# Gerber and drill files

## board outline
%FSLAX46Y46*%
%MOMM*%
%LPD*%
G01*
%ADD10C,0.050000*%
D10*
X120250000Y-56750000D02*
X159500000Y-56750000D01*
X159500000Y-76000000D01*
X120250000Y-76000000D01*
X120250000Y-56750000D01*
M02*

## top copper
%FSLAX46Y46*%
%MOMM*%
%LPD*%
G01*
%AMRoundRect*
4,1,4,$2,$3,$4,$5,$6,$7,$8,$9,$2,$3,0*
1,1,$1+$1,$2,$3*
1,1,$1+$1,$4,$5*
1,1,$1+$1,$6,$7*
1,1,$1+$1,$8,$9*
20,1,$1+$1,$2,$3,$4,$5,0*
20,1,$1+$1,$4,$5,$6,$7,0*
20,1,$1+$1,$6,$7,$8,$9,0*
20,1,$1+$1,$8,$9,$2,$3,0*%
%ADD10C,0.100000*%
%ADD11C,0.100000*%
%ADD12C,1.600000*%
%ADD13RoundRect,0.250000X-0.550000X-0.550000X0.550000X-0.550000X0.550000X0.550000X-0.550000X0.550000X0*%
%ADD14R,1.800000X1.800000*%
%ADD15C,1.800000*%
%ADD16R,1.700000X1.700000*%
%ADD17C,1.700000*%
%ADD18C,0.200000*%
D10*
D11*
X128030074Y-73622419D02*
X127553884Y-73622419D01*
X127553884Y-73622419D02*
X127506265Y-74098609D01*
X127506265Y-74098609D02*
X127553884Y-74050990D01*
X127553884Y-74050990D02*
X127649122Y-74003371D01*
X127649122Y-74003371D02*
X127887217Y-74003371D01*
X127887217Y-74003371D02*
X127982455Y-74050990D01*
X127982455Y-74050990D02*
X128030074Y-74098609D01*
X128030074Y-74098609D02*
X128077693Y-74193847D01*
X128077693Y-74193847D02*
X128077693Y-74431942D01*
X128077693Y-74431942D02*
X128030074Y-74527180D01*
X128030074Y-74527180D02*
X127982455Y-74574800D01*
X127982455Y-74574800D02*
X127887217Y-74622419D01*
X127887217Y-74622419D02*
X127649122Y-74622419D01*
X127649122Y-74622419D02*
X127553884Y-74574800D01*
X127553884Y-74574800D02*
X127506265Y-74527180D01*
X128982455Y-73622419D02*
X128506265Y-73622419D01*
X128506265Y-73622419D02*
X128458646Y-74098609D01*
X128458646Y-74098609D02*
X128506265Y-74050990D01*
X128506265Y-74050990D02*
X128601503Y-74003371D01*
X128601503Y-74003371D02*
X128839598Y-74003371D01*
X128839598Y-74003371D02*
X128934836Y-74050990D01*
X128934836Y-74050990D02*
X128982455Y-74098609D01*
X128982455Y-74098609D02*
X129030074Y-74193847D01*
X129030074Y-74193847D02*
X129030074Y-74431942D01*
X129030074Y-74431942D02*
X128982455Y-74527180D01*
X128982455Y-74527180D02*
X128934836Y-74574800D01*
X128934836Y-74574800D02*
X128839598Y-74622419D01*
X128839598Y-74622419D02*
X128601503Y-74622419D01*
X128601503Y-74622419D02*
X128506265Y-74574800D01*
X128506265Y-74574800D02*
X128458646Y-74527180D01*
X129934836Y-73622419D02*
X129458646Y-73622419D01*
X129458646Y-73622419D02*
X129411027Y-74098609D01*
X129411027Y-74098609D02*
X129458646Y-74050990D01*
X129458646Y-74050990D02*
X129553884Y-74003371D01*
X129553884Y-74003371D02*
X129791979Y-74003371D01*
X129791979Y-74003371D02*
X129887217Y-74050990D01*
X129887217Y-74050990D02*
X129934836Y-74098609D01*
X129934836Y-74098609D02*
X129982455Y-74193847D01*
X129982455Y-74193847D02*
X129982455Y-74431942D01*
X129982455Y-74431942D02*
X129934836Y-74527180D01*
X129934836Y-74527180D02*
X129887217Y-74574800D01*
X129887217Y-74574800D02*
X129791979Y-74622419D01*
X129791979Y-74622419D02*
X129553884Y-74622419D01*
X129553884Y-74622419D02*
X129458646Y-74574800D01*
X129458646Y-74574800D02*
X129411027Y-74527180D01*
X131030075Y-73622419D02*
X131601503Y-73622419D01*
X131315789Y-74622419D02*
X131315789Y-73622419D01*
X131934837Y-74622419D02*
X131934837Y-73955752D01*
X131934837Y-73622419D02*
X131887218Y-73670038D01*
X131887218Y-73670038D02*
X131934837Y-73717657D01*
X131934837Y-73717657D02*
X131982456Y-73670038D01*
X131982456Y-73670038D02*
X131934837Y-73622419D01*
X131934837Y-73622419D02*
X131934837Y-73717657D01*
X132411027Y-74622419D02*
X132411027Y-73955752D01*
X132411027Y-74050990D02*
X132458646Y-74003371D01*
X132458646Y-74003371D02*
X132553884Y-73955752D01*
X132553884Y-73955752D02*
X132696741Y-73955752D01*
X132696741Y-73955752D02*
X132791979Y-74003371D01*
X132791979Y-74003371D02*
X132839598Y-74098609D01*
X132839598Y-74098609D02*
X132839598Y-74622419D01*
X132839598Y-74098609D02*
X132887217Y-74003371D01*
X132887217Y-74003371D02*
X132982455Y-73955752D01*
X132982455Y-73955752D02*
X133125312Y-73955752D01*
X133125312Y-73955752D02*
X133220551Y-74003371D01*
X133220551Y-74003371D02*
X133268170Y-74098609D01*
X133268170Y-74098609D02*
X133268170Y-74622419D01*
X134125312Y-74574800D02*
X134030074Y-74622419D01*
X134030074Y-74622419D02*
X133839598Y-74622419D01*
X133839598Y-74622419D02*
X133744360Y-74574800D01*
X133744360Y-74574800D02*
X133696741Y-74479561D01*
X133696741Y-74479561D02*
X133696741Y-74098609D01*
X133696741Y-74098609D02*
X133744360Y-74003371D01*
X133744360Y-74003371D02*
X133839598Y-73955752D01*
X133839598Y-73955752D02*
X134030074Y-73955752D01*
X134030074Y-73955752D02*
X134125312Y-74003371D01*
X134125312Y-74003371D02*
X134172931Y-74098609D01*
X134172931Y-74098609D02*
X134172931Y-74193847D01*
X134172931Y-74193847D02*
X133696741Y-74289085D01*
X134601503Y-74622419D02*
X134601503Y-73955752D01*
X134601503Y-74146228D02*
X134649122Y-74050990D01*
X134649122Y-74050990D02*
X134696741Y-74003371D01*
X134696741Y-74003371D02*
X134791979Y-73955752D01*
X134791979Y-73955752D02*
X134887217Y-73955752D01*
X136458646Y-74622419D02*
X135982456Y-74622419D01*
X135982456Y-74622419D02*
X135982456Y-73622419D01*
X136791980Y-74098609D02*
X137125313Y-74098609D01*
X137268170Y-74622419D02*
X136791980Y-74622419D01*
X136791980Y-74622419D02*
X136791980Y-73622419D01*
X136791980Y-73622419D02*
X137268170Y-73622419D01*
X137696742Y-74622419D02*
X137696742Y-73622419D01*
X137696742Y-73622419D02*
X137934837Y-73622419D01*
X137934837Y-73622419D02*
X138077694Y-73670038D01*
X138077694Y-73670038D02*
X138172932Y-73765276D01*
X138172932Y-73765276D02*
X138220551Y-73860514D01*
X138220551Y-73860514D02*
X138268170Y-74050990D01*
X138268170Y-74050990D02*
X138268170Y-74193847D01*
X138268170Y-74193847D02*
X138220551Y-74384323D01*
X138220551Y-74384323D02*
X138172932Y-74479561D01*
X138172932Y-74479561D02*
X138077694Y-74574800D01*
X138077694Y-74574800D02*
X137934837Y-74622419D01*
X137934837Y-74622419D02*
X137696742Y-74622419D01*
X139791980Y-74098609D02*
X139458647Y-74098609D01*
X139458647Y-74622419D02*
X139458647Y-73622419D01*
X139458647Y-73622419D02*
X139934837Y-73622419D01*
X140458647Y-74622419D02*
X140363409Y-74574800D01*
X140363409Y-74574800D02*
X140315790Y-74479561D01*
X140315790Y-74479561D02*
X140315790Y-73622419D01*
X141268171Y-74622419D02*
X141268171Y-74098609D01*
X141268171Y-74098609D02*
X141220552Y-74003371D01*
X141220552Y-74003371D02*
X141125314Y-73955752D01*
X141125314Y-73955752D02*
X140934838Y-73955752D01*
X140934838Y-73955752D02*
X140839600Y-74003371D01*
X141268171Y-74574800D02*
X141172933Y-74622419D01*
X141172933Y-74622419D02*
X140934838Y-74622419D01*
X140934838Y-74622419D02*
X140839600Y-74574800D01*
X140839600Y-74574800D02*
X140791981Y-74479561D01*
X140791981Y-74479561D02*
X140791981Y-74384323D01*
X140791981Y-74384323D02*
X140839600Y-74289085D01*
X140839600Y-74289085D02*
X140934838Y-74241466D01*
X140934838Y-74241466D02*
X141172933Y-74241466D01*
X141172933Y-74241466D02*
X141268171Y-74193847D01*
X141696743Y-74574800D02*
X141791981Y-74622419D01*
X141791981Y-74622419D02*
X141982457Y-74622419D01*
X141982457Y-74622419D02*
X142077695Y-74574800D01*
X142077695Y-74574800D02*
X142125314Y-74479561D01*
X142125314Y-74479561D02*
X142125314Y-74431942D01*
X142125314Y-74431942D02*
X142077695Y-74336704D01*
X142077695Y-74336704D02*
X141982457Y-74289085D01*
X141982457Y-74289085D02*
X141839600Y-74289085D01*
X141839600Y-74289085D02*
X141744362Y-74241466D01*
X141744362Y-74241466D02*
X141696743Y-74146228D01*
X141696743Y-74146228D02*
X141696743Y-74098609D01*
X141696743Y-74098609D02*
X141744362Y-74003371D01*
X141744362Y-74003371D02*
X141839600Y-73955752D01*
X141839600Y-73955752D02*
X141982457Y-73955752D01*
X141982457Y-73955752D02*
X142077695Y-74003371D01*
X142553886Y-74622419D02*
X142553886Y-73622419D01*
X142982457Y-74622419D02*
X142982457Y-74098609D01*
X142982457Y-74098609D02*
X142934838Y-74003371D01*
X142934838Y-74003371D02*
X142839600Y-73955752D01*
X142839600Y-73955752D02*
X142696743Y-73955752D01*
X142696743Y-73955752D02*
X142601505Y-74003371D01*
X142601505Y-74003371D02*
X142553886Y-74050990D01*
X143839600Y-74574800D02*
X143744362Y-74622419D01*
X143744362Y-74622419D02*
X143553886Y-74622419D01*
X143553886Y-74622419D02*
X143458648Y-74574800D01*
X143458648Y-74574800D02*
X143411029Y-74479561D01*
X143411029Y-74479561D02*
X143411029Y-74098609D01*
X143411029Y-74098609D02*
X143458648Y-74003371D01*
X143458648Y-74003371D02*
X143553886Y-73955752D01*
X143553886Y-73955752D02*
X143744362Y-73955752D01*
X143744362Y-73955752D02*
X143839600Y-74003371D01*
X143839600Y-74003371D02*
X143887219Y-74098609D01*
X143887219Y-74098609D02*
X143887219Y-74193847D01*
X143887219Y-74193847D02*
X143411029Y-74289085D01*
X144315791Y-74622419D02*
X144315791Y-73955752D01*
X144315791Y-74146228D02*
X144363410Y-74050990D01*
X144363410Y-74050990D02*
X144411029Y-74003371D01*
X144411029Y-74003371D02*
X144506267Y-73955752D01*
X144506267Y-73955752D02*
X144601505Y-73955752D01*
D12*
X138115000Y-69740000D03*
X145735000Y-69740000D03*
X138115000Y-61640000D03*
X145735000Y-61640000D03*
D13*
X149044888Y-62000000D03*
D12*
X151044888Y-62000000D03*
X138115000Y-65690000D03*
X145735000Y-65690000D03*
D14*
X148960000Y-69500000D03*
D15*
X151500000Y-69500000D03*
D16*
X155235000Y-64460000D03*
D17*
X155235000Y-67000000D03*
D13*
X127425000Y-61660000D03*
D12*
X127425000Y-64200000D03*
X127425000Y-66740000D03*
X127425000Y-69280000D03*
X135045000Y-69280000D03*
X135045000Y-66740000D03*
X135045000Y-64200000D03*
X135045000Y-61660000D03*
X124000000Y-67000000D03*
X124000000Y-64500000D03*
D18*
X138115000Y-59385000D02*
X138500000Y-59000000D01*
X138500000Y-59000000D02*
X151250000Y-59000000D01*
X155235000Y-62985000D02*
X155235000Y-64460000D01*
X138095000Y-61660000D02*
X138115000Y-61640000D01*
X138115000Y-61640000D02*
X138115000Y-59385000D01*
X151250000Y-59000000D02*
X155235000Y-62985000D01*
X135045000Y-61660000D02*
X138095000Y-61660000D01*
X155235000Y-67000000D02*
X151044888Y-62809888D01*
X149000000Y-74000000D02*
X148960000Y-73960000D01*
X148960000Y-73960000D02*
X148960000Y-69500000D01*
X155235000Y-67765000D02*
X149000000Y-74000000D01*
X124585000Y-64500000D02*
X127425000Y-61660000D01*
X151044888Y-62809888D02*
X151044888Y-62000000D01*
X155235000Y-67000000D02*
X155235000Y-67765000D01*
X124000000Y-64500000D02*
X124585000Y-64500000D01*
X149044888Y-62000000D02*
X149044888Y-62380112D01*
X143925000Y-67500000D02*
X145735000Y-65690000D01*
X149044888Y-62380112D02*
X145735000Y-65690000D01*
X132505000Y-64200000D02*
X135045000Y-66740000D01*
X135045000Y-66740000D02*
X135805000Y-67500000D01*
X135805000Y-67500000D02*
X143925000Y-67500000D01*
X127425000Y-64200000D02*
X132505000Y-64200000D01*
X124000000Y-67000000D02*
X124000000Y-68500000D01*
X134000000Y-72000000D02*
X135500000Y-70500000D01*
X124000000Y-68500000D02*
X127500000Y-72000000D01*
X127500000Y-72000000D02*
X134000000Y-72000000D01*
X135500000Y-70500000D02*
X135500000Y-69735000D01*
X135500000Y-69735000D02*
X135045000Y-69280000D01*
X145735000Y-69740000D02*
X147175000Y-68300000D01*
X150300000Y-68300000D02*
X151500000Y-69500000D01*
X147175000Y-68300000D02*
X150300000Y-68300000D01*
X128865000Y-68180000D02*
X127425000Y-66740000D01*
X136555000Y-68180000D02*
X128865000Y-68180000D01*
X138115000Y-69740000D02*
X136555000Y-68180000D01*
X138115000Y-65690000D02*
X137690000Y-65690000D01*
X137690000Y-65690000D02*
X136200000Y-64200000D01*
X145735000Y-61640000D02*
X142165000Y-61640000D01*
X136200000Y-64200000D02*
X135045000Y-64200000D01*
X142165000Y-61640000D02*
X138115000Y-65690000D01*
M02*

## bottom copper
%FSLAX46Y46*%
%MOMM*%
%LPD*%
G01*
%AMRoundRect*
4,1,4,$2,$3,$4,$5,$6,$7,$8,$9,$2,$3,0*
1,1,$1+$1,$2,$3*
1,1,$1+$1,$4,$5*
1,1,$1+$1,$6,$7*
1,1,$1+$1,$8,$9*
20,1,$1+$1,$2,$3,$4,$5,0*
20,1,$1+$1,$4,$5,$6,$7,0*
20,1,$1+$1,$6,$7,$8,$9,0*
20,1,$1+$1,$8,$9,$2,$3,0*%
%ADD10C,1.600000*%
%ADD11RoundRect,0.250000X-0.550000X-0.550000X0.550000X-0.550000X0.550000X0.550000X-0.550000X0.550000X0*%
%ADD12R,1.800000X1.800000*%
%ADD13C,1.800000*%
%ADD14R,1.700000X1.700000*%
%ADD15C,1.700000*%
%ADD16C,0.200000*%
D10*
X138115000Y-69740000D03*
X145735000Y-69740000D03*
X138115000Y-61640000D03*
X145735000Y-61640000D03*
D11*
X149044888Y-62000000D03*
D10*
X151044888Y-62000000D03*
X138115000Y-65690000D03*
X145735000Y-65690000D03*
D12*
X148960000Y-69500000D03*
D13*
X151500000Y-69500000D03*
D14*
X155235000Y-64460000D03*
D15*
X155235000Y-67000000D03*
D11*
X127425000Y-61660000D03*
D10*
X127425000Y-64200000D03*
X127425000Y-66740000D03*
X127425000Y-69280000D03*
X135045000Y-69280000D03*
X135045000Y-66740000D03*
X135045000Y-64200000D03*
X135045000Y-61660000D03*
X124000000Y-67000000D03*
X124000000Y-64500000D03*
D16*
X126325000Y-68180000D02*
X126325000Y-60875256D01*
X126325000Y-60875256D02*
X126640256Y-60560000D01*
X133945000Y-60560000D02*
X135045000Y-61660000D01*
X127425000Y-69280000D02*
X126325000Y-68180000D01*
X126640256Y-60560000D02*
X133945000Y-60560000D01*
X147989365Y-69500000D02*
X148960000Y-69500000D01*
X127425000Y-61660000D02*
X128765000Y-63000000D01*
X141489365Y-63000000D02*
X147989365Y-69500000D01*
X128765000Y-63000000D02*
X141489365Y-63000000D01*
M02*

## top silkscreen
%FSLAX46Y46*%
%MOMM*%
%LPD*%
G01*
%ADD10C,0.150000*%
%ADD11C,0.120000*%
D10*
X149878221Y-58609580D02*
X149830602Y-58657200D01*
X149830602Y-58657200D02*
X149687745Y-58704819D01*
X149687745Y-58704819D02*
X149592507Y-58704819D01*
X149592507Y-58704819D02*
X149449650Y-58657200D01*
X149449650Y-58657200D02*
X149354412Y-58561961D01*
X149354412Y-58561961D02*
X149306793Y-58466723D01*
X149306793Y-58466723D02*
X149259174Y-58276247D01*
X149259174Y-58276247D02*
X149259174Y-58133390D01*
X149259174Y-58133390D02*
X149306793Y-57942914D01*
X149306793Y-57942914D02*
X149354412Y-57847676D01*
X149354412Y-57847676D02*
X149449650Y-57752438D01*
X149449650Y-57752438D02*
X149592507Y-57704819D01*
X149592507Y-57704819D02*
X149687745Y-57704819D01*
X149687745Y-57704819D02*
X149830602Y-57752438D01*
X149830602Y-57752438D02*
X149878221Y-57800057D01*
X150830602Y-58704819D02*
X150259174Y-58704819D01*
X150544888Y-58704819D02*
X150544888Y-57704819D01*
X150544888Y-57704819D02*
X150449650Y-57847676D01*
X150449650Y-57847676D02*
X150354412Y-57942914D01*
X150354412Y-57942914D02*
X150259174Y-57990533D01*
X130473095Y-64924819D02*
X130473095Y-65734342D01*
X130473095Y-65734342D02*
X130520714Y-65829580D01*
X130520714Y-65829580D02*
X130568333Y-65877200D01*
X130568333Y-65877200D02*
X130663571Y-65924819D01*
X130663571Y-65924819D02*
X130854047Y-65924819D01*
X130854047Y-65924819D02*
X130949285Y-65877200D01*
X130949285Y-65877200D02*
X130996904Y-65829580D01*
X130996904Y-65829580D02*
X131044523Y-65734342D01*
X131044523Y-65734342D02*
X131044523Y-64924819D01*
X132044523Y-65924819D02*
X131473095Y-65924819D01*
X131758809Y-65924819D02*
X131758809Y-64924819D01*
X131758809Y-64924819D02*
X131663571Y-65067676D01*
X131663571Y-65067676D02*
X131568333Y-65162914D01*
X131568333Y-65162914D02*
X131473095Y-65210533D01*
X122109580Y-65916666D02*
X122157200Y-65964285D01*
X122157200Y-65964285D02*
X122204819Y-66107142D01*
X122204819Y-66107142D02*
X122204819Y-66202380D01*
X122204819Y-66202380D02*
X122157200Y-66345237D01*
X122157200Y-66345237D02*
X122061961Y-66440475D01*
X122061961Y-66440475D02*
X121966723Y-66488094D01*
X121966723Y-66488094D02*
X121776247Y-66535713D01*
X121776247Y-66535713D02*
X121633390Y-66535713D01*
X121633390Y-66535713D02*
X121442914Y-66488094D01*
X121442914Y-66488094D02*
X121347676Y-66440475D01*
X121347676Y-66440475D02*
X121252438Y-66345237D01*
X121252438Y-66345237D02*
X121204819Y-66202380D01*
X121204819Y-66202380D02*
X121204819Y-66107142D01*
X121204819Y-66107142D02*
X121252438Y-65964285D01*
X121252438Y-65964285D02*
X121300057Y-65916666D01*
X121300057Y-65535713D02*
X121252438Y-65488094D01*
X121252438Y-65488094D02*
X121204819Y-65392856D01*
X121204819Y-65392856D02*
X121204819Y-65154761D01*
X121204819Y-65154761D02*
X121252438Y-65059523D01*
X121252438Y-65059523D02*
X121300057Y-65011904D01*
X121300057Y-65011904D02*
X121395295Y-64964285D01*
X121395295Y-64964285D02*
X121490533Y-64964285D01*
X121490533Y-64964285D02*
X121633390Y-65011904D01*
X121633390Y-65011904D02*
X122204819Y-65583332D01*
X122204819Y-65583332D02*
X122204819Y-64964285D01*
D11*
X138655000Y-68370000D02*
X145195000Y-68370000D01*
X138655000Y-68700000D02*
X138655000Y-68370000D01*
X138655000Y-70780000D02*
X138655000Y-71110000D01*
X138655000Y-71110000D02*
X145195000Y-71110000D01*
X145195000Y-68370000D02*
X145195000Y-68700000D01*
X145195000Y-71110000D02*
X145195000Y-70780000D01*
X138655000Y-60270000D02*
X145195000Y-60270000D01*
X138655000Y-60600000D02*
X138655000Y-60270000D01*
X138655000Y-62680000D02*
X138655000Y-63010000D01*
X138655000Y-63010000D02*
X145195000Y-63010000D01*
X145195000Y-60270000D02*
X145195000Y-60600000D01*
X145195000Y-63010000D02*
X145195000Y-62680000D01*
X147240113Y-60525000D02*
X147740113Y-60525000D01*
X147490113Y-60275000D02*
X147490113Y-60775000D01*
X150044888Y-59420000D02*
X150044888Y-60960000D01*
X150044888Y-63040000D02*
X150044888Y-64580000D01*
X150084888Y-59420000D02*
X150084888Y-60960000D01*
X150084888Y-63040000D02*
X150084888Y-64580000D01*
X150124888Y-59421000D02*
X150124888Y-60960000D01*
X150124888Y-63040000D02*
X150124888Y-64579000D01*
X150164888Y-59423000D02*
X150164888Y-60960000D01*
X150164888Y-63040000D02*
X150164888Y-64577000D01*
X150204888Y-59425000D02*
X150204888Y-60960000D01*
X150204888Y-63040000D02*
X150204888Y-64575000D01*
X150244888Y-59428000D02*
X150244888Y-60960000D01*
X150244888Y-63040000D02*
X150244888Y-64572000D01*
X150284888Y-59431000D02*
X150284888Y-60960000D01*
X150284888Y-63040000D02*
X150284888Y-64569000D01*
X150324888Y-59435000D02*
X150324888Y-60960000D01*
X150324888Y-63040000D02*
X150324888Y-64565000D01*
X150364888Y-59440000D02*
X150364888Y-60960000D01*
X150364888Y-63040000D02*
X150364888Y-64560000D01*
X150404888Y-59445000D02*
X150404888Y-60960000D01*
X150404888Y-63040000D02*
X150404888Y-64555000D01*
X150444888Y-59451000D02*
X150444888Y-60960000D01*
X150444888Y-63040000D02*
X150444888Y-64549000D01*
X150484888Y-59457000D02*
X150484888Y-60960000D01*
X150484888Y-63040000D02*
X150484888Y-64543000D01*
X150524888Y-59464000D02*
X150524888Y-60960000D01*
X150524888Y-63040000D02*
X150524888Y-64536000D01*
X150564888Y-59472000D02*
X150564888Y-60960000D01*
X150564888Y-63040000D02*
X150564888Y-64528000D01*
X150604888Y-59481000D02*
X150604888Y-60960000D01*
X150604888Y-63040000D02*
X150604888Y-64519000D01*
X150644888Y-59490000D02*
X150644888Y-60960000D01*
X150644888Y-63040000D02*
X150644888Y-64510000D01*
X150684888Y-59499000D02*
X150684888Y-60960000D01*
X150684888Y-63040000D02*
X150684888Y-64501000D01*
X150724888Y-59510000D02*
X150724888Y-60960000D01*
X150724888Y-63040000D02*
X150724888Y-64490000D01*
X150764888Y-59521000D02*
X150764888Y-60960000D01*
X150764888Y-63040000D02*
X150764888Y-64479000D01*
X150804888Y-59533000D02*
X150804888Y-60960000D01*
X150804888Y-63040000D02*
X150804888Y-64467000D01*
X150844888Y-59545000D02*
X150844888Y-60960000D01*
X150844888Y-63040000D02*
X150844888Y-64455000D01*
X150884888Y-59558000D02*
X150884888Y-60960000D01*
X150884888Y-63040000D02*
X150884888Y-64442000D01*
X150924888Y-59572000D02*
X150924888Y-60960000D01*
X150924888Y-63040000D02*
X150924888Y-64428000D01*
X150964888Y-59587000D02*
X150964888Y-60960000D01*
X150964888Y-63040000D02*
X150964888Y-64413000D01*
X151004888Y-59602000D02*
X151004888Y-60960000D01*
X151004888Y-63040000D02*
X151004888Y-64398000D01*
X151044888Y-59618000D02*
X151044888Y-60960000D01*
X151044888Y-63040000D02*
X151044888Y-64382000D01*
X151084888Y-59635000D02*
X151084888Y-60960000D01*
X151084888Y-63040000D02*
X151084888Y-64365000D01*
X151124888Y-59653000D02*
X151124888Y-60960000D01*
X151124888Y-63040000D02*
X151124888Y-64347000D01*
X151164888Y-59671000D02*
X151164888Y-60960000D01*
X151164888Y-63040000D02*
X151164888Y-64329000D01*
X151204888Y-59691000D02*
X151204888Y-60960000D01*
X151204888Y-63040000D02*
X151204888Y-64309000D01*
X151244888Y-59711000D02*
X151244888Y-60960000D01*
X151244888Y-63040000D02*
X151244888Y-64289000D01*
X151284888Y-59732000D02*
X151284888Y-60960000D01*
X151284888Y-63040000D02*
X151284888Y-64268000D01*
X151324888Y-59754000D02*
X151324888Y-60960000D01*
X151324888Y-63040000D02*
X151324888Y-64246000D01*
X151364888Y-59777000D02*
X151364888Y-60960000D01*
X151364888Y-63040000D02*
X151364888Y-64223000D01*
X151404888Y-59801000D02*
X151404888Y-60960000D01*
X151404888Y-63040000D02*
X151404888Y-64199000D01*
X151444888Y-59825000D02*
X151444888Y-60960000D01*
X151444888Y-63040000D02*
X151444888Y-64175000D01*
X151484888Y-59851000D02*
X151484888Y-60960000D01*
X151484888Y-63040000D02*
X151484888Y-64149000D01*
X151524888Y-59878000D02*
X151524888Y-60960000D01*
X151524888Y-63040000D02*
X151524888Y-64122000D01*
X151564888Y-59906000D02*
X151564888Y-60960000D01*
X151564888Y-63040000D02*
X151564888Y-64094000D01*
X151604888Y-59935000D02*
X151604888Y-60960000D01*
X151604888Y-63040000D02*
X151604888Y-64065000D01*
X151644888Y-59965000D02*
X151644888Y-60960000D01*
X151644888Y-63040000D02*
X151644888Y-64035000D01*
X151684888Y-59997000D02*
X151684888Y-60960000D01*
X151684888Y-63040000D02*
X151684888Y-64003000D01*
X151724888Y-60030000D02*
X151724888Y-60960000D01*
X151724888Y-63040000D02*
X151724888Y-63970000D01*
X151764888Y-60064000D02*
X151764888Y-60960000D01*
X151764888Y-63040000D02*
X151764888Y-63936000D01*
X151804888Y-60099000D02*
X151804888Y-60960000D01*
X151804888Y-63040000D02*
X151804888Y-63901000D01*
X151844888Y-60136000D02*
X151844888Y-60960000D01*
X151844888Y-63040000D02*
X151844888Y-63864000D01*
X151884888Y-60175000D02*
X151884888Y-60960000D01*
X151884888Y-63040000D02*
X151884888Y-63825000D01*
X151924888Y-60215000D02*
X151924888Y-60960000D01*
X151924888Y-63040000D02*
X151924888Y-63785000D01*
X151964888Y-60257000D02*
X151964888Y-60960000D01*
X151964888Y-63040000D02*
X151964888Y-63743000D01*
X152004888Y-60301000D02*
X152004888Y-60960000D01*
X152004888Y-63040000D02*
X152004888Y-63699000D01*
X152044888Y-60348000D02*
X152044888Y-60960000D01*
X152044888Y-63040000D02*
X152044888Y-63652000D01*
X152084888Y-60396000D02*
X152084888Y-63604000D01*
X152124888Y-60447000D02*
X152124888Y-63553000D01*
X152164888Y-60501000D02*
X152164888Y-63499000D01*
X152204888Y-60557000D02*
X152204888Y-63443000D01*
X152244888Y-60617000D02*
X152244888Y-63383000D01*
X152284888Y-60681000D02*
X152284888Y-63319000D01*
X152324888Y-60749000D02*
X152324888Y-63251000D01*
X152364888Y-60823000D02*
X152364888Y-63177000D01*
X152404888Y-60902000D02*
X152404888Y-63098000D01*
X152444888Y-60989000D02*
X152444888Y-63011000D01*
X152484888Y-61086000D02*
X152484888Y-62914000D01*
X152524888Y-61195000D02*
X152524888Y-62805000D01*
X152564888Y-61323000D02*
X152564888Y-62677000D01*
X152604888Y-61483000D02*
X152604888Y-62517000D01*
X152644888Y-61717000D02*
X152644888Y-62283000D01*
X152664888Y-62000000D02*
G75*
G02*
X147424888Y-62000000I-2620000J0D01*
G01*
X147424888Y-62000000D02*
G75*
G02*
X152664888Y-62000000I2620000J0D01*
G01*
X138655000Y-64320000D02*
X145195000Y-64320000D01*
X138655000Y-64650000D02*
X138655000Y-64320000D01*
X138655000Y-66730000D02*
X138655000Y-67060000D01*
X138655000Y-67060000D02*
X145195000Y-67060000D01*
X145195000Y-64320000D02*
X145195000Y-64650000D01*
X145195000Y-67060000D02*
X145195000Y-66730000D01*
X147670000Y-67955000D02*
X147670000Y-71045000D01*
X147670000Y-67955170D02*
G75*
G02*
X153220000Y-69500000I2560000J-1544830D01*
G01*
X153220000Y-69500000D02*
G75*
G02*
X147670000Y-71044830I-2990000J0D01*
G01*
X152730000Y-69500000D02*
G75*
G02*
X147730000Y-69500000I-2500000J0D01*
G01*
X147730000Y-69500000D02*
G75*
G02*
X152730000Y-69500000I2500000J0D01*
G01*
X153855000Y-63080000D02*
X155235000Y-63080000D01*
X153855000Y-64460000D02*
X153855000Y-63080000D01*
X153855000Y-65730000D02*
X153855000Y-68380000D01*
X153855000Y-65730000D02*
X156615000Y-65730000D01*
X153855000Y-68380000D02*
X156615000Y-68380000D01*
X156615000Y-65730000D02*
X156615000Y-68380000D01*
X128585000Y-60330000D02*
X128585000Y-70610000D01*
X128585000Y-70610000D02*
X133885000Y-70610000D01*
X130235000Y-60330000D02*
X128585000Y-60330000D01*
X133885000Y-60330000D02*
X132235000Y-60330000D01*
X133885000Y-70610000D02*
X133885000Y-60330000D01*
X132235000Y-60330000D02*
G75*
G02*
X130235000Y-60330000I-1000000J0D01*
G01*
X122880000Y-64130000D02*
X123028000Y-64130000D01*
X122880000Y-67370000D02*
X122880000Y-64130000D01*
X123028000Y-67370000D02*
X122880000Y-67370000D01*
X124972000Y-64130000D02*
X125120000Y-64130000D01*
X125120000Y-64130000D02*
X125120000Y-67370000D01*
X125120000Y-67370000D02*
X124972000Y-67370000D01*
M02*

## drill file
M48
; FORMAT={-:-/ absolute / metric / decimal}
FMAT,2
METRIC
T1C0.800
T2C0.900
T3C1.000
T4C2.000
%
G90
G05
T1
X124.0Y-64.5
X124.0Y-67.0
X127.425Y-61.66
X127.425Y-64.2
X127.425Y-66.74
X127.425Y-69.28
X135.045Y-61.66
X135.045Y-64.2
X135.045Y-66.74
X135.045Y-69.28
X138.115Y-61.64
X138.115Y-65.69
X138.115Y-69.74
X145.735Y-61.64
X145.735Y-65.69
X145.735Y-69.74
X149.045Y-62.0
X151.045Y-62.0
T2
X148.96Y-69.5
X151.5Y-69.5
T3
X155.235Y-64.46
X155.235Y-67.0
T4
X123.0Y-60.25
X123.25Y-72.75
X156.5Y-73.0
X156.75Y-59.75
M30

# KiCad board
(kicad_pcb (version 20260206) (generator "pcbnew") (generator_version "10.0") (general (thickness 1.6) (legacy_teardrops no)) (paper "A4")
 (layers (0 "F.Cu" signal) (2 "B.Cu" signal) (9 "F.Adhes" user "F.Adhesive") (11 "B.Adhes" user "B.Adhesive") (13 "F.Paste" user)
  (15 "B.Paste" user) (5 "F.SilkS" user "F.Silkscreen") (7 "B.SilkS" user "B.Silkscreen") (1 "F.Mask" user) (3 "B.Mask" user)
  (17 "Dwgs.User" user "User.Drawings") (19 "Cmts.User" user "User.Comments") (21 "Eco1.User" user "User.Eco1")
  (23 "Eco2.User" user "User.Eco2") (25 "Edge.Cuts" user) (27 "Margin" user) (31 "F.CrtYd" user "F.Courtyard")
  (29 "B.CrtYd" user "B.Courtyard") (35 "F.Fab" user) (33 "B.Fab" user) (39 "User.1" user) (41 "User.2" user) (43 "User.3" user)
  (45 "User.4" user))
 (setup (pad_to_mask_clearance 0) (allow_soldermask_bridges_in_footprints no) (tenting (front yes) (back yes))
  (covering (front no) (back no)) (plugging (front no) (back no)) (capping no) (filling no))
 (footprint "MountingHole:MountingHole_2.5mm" (layer "F.Cu") (at 123.25 72.75)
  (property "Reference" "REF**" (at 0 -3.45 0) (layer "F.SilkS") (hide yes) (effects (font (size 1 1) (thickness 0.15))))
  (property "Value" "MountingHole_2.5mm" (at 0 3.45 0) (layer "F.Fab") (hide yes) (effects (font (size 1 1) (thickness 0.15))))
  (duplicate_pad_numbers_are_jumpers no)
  (pad "" np_thru_hole circle (at 0 0) (size 0.5 0.5) (drill 2) (layers "*.Cu" "*.Mask")))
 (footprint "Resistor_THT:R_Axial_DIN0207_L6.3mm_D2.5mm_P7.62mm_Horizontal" (layer "F.Cu") (at 138.115 69.74)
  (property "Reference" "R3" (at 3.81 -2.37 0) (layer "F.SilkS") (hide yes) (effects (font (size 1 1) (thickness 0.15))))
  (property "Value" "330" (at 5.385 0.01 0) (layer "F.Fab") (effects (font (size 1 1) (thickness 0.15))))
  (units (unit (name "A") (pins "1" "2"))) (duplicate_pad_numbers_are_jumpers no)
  (fp_line (start 0.54 -1.37) (end 7.08 -1.37) (stroke (width 0.12) (type solid)) (layer "F.SilkS"))
  (fp_line (start 0.54 -1.04) (end 0.54 -1.37) (stroke (width 0.12) (type solid)) (layer "F.SilkS"))
  (fp_line (start 0.54 1.04) (end 0.54 1.37) (stroke (width 0.12) (type solid)) (layer "F.SilkS"))
  (fp_line (start 0.54 1.37) (end 7.08 1.37) (stroke (width 0.12) (type solid)) (layer "F.SilkS"))
  (fp_line (start 7.08 -1.37) (end 7.08 -1.04) (stroke (width 0.12) (type solid)) (layer "F.SilkS"))
  (fp_line (start 7.08 1.37) (end 7.08 1.04) (stroke (width 0.12) (type solid)) (layer "F.SilkS"))
  (pad "1" thru_hole circle (at 0 0) (size 1.6 1.6) (drill 0.8) (layers "*.Cu" "*.Mask") (remove_unused_layers no) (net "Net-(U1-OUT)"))
  (pad "2" thru_hole circle (at 7.62 0) (size 1.6 1.6) (drill 0.8) (layers "*.Cu" "*.Mask") (remove_unused_layers no) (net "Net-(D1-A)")))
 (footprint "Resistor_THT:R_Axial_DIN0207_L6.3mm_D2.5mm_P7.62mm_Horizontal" (layer "F.Cu") (at 138.115 61.64)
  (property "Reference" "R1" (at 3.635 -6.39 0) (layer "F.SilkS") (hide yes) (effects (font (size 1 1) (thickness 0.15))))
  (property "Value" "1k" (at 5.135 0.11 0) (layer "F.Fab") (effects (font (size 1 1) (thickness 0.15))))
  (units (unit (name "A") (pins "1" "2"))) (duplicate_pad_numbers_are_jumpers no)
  (fp_line (start 0.54 -1.37) (end 7.08 -1.37) (stroke (width 0.12) (type solid)) (layer "F.SilkS"))
  (fp_line (start 0.54 -1.04) (end 0.54 -1.37) (stroke (width 0.12) (type solid)) (layer "F.SilkS"))
  (fp_line (start 0.54 1.04) (end 0.54 1.37) (stroke (width 0.12) (type solid)) (layer "F.SilkS"))
  (fp_line (start 0.54 1.37) (end 7.08 1.37) (stroke (width 0.12) (type solid)) (layer "F.SilkS"))
  (fp_line (start 7.08 -1.37) (end 7.08 -1.04) (stroke (width 0.12) (type solid)) (layer "F.SilkS"))
  (fp_line (start 7.08 1.37) (end 7.08 1.04) (stroke (width 0.12) (type solid)) (layer "F.SilkS"))
  (pad "1" thru_hole circle (at 0 0) (size 1.6 1.6) (drill 0.8) (layers "*.Cu" "*.Mask") (remove_unused_layers no) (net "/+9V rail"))
  (pad "2" thru_hole circle (at 7.62 0) (size 1.6 1.6) (drill 0.8) (layers "*.Cu" "*.Mask") (remove_unused_layers no) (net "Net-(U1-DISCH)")))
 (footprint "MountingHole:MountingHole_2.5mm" (layer "F.Cu") (at 156.75 59.75)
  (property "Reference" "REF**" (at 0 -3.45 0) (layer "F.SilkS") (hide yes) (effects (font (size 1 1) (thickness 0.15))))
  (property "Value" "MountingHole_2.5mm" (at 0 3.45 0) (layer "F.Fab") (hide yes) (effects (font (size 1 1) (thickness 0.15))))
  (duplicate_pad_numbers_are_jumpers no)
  (pad "" np_thru_hole circle (at 0 0) (size 0.5 0.5) (drill 2) (layers "*.Cu" "*.Mask")))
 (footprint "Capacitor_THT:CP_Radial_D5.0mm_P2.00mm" (layer "F.Cu") (at 149.044888 62)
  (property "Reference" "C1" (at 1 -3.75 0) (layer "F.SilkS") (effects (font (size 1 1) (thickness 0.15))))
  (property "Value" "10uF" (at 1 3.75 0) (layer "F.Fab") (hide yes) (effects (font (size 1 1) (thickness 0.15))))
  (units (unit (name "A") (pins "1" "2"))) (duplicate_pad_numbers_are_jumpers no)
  (fp_line (start -1.804775 -1.475) (end -1.304775 -1.475) (stroke (width 0.12) (type solid)) (layer "F.SilkS"))
  (fp_line (start -1.554775 -1.725) (end -1.554775 -1.225) (stroke (width 0.12) (type solid)) (layer "F.SilkS"))
  (fp_line (start 1 -2.58) (end 1 -1.04) (stroke (width 0.12) (type solid)) (layer "F.SilkS"))
  (fp_line (start 1 1.04) (end 1 2.58) (stroke (width 0.12) (type solid)) (layer "F.SilkS"))
  (fp_line (start 1.04 -2.58) (end 1.04 -1.04) (stroke (width 0.12) (type solid)) (layer "F.SilkS"))
  (fp_line (start 1.04 1.04) (end 1.04 2.58) (stroke (width 0.12) (type solid)) (layer "F.SilkS"))
  (fp_line (start 1.08 -2.579) (end 1.08 -1.04) (stroke (width 0.12) (type solid)) (layer "F.SilkS"))
  (fp_line (start 1.08 1.04) (end 1.08 2.579) (stroke (width 0.12) (type solid)) (layer "F.SilkS"))
  (fp_line (start 1.12 -2.577) (end 1.12 -1.04) (stroke (width 0.12) (type solid)) (layer "F.SilkS"))
  (fp_line (start 1.12 1.04) (end 1.12 2.577) (stroke (width 0.12) (type solid)) (layer "F.SilkS"))
  (fp_line (start 1.16 -2.575) (end 1.16 -1.04) (stroke (width 0.12) (type solid)) (layer "F.SilkS"))
  (fp_line (start 1.16 1.04) (end 1.16 2.575) (stroke (width 0.12) (type solid)) (layer "F.SilkS"))
  (fp_line (start 1.2 -2.572) (end 1.2 -1.04) (stroke (width 0.12) (type solid)) (layer "F.SilkS"))
  (fp_line (start 1.2 1.04) (end 1.2 2.572) (stroke (width 0.12) (type solid)) (layer "F.SilkS"))
  (fp_line (start 1.24 -2.569) (end 1.24 -1.04) (stroke (width 0.12) (type solid)) (layer "F.SilkS"))
  (fp_line (start 1.24 1.04) (end 1.24 2.569) (stroke (width 0.12) (type solid)) (layer "F.SilkS"))
  (fp_line (start 1.28 -2.565) (end 1.28 -1.04) (stroke (width 0.12) (type solid)) (layer "F.SilkS"))
  (fp_line (start 1.28 1.04) (end 1.28 2.565) (stroke (width 0.12) (type solid)) (layer "F.SilkS"))
  (fp_line (start 1.32 -2.56) (end 1.32 -1.04) (stroke (width 0.12) (type solid)) (layer "F.SilkS"))
  (fp_line (start 1.32 1.04) (end 1.32 2.56) (stroke (width 0.12) (type solid)) (layer "F.SilkS"))
  (fp_line (start 1.36 -2.555) (end 1.36 -1.04) (stroke (width 0.12) (type solid)) (layer "F.SilkS"))
  (fp_line (start 1.36 1.04) (end 1.36 2.555) (stroke (width 0.12) (type solid)) (layer "F.SilkS"))
  (fp_line (start 1.4 -2.549) (end 1.4 -1.04) (stroke (width 0.12) (type solid)) (layer "F.SilkS"))
  (fp_line (start 1.4 1.04) (end 1.4 2.549) (stroke (width 0.12) (type solid)) (layer "F.SilkS"))
  (fp_line (start 1.44 -2.543) (end 1.44 -1.04) (stroke (width 0.12) (type solid)) (layer "F.SilkS"))
  (fp_line (start 1.44 1.04) (end 1.44 2.543) (stroke (width 0.12) (type solid)) (layer "F.SilkS"))
  (fp_line (start 1.48 -2.536) (end 1.48 -1.04) (stroke (width 0.12) (type solid)) (layer "F.SilkS"))
  (fp_line (start 1.48 1.04) (end 1.48 2.536) (stroke (width 0.12) (type solid)) (layer "F.SilkS"))
  (fp_line (start 1.52 -2.528) (end 1.52 -1.04) (stroke (width 0.12) (type solid)) (layer "F.SilkS"))
  (fp_line (start 1.52 1.04) (end 1.52 2.528) (stroke (width 0.12) (type solid)) (layer "F.SilkS"))
  (fp_line (start 1.56 -2.519) (end 1.56 -1.04) (stroke (width 0.12) (type solid)) (layer "F.SilkS"))
  (fp_line (start 1.56 1.04) (end 1.56 2.519) (stroke (width 0.12) (type solid)) (layer "F.SilkS"))
  (fp_line (start 1.6 -2.51) (end 1.6 -1.04) (stroke (width 0.12) (type solid)) (layer "F.SilkS"))
  (fp_line (start 1.6 1.04) (end 1.6 2.51) (stroke (width 0.12) (type solid)) (layer "F.SilkS"))
  (fp_line (start 1.64 -2.501) (end 1.64 -1.04) (stroke (width 0.12) (type solid)) (layer "F.SilkS"))
  (fp_line (start 1.64 1.04) (end 1.64 2.501) (stroke (width 0.12) (type solid)) (layer "F.SilkS"))
  (fp_line (start 1.68 -2.49) (end 1.68 -1.04) (stroke (width 0.12) (type solid)) (layer "F.SilkS"))
  (fp_line (start 1.68 1.04) (end 1.68 2.49) (stroke (width 0.12) (type solid)) (layer "F.SilkS"))
  (fp_line (start 1.72 -2.479) (end 1.72 -1.04) (stroke (width 0.12) (type solid)) (layer "F.SilkS"))
  (fp_line (start 1.72 1.04) (end 1.72 2.479) (stroke (width 0.12) (type solid)) (layer "F.SilkS"))
  (fp_line (start 1.76 -2.467) (end 1.76 -1.04) (stroke (width 0.12) (type solid)) (layer "F.SilkS"))
  (fp_line (start 1.76 1.04) (end 1.76 2.467) (stroke (width 0.12) (type solid)) (layer "F.SilkS"))
  (fp_line (start 1.8 -2.455) (end 1.8 -1.04) (stroke (width 0.12) (type solid)) (layer "F.SilkS"))
  (fp_line (start 1.8 1.04) (end 1.8 2.455) (stroke (width 0.12) (type solid)) (layer "F.SilkS"))
  (fp_line (start 1.84 -2.442) (end 1.84 -1.04) (stroke (width 0.12) (type solid)) (layer "F.SilkS"))
  (fp_line (start 1.84 1.04) (end 1.84 2.442) (stroke (width 0.12) (type solid)) (layer "F.SilkS"))
  (fp_line (start 1.88 -2.428) (end 1.88 -1.04) (stroke (width 0.12) (type solid)) (layer "F.SilkS"))
  (fp_line (start 1.88 1.04) (end 1.88 2.428) (stroke (width 0.12) (type solid)) (layer "F.SilkS"))
  (fp_line (start 1.92 -2.413) (end 1.92 -1.04) (stroke (width 0.12) (type solid)) (layer "F.SilkS"))
  (fp_line (start 1.92 1.04) (end 1.92 2.413) (stroke (width 0.12) (type solid)) (layer "F.SilkS"))
  (fp_line (start 1.96 -2.398) (end 1.96 -1.04) (stroke (width 0.12) (type solid)) (layer "F.SilkS"))
  (fp_line (start 1.96 1.04) (end 1.96 2.398) (stroke (width 0.12) (type solid)) (layer "F.SilkS"))
  (fp_line (start 2 -2.382) (end 2 -1.04) (stroke (width 0.12) (type solid)) (layer "F.SilkS"))
  (fp_line (start 2 1.04) (end 2 2.382) (stroke (width 0.12) (type solid)) (layer "F.SilkS"))
  (fp_line (start 2.04 -2.365) (end 2.04 -1.04) (stroke (width 0.12) (type solid)) (layer "F.SilkS"))
  (fp_line (start 2.04 1.04) (end 2.04 2.365) (stroke (width 0.12) (type solid)) (layer "F.SilkS"))
  (fp_line (start 2.08 -2.347) (end 2.08 -1.04) (stroke (width 0.12) (type solid)) (layer "F.SilkS"))
  (fp_line (start 2.08 1.04) (end 2.08 2.347) (stroke (width 0.12) (type solid)) (layer "F.SilkS"))
  (fp_line (start 2.12 -2.329) (end 2.12 -1.04) (stroke (width 0.12) (type solid)) (layer "F.SilkS"))
  (fp_line (start 2.12 1.04) (end 2.12 2.329) (stroke (width 0.12) (type solid)) (layer "F.SilkS"))
  (fp_line (start 2.16 -2.309) (end 2.16 -1.04) (stroke (width 0.12) (type solid)) (layer "F.SilkS"))
  (fp_line (start 2.16 1.04) (end 2.16 2.309) (stroke (width 0.12) (type solid)) (layer "F.SilkS"))
  (fp_line (start 2.2 -2.289) (end 2.2 -1.04) (stroke (width 0.12) (type solid)) (layer "F.SilkS"))
  (fp_line (start 2.2 1.04) (end 2.2 2.289) (stroke (width 0.12) (type solid)) (layer "F.SilkS"))
  (fp_line (start 2.24 -2.268) (end 2.24 -1.04) (stroke (width 0.12) (type solid)) (layer "F.SilkS"))
  (fp_line (start 2.24 1.04) (end 2.24 2.268) (stroke (width 0.12) (type solid)) (layer "F.SilkS"))
  (fp_line (start 2.28 -2.246) (end 2.28 -1.04) (stroke (width 0.12) (type solid)) (layer "F.SilkS"))
  (fp_line (start 2.28 1.04) (end 2.28 2.246) (stroke (width 0.12) (type solid)) (layer "F.SilkS"))
  (fp_line (start 2.32 -2.223) (end 2.32 -1.04) (stroke (width 0.12) (type solid)) (layer "F.SilkS"))
  (fp_line (start 2.32 1.04) (end 2.32 2.223) (stroke (width 0.12) (type solid)) (layer "F.SilkS"))
  (fp_line (start 2.36 -2.199) (end 2.36 -1.04) (stroke (width 0.12) (type solid)) (layer "F.SilkS"))
  (fp_line (start 2.36 1.04) (end 2.36 2.199) (stroke (width 0.12) (type solid)) (layer "F.SilkS"))
  (fp_line (start 2.4 -2.175) (end 2.4 -1.04) (stroke (width 0.12) (type solid)) (layer "F.SilkS"))
  (fp_line (start 2.4 1.04) (end 2.4 2.175) (stroke (width 0.12) (type solid)) (layer "F.SilkS"))
  (fp_line (start 2.44 -2.149) (end 2.44 -1.04) (stroke (width 0.12) (type solid)) (layer "F.SilkS"))
  (fp_line (start 2.44 1.04) (end 2.44 2.149) (stroke (width 0.12) (type solid)) (layer "F.SilkS"))
  (fp_line (start 2.48 -2.122) (end 2.48 -1.04) (stroke (width 0.12) (type solid)) (layer "F.SilkS"))
  (fp_line (start 2.48 1.04) (end 2.48 2.122) (stroke (width 0.12) (type solid)) (layer "F.SilkS"))
  (fp_line (start 2.52 -2.094) (end 2.52 -1.04) (stroke (width 0.12) (type solid)) (layer "F.SilkS"))
  (fp_line (start 2.52 1.04) (end 2.52 2.094) (stroke (width 0.12) (type solid)) (layer "F.SilkS"))
  (fp_line (start 2.56 -2.065) (end 2.56 -1.04) (stroke (width 0.12) (type solid)) (layer "F.SilkS"))
  (fp_line (start 2.56 1.04) (end 2.56 2.065) (stroke (width 0.12) (type solid)) (layer "F.SilkS"))
  (fp_line (start 2.6 -2.035) (end 2.6 -1.04) (stroke (width 0.12) (type solid)) (layer "F.SilkS"))
  (fp_line (start 2.6 1.04) (end 2.6 2.035) (stroke (width 0.12) (type solid)) (layer "F.SilkS"))
  (fp_line (start 2.64 -2.003) (end 2.64 -1.04) (stroke (width 0.12) (type solid)) (layer "F.SilkS"))
  (fp_line (start 2.64 1.04) (end 2.64 2.003) (stroke (width 0.12) (type solid)) (layer "F.SilkS"))
  (fp_line (start 2.68 -1.97) (end 2.68 -1.04) (stroke (width 0.12) (type solid)) (layer "F.SilkS"))
  (fp_line (start 2.68 1.04) (end 2.68 1.97) (stroke (width 0.12) (type solid)) (layer "F.SilkS"))
  (fp_line (start 2.72 -1.936) (end 2.72 -1.04) (stroke (width 0.12) (type solid)) (layer "F.SilkS"))
  (fp_line (start 2.72 1.04) (end 2.72 1.936) (stroke (width 0.12) (type solid)) (layer "F.SilkS"))
  (fp_line (start 2.76 -1.901) (end 2.76 -1.04) (stroke (width 0.12) (type solid)) (layer "F.SilkS"))
  (fp_line (start 2.76 1.04) (end 2.76 1.901) (stroke (width 0.12) (type solid)) (layer "F.SilkS"))
  (fp_line (start 2.8 -1.864) (end 2.8 -1.04) (stroke (width 0.12) (type solid)) (layer "F.SilkS"))
  (fp_line (start 2.8 1.04) (end 2.8 1.864) (stroke (width 0.12) (type solid)) (layer "F.SilkS"))
  (fp_line (start 2.84 -1.825) (end 2.84 -1.04) (stroke (width 0.12) (type solid)) (layer "F.SilkS"))
  (fp_line (start 2.84 1.04) (end 2.84 1.825) (stroke (width 0.12) (type solid)) (layer "F.SilkS"))
  (fp_line (start 2.88 -1.785) (end 2.88 -1.04) (stroke (width 0.12) (type solid)) (layer "F.SilkS"))
  (fp_line (start 2.88 1.04) (end 2.88 1.785) (stroke (width 0.12) (type solid)) (layer "F.SilkS"))
  (fp_line (start 2.92 -1.743) (end 2.92 -1.04) (stroke (width 0.12) (type solid)) (layer "F.SilkS"))
  (fp_line (start 2.92 1.04) (end 2.92 1.743) (stroke (width 0.12) (type solid)) (layer "F.SilkS"))
  (fp_line (start 2.96 -1.699) (end 2.96 -1.04) (stroke (width 0.12) (type solid)) (layer "F.SilkS"))
  (fp_line (start 2.96 1.04) (end 2.96 1.699) (stroke (width 0.12) (type solid)) (layer "F.SilkS"))
  (fp_line (start 3 -1.652) (end 3 -1.04) (stroke (width 0.12) (type solid)) (layer "F.SilkS"))
  (fp_line (start 3 1.04) (end 3 1.652) (stroke (width 0.12) (type solid)) (layer "F.SilkS"))
  (fp_line (start 3.04 -1.604) (end 3.04 1.604) (stroke (width 0.12) (type solid)) (layer "F.SilkS"))
  (fp_line (start 3.08 -1.553) (end 3.08 1.553) (stroke (width 0.12) (type solid)) (layer "F.SilkS"))
  (fp_line (start 3.12 -1.499) (end 3.12 1.499) (stroke (width 0.12) (type solid)) (layer "F.SilkS"))
  (fp_line (start 3.16 -1.443) (end 3.16 1.443) (stroke (width 0.12) (type solid)) (layer "F.SilkS"))
  (fp_line (start 3.2 -1.383) (end 3.2 1.383) (stroke (width 0.12) (type solid)) (layer "F.SilkS"))
  (fp_line (start 3.24 -1.319) (end 3.24 1.319) (stroke (width 0.12) (type solid)) (layer "F.SilkS"))
  (fp_line (start 3.28 -1.251) (end 3.28 1.251) (stroke (width 0.12) (type solid)) (layer "F.SilkS"))
  (fp_line (start 3.32 -1.177) (end 3.32 1.177) (stroke (width 0.12) (type solid)) (layer "F.SilkS"))
  (fp_line (start 3.36 -1.098) (end 3.36 1.098) (stroke (width 0.12) (type solid)) (layer "F.SilkS"))
  (fp_line (start 3.4 -1.011) (end 3.4 1.011) (stroke (width 0.12) (type solid)) (layer "F.SilkS"))
  (fp_line (start 3.44 -0.914) (end 3.44 0.914) (stroke (width 0.12) (type solid)) (layer "F.SilkS"))
  (fp_line (start 3.48 -0.805) (end 3.48 0.805) (stroke (width 0.12) (type solid)) (layer "F.SilkS"))
  (fp_line (start 3.52 -0.677) (end 3.52 0.677) (stroke (width 0.12) (type solid)) (layer "F.SilkS"))
  (fp_line (start 3.56 -0.517) (end 3.56 0.517) (stroke (width 0.12) (type solid)) (layer "F.SilkS"))
  (fp_line (start 3.6 -0.283) (end 3.6 0.283) (stroke (width 0.12) (type solid)) (layer "F.SilkS"))
  (fp_circle (center 1 0) (end 3.62 0) (stroke (width 0.12) (type solid)) (fill no) (layer "F.SilkS"))
  (pad "1" thru_hole roundrect (at 0 0) (size 1.6 1.6) (drill 0.8) (layers "*.Cu" "*.Mask") (remove_unused_layers no)
   (roundrect_rratio 0.15625) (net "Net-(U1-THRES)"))
  (pad "2" thru_hole circle (at 2 0) (size 1.6 1.6) (drill 0.8) (layers "*.Cu" "*.Mask") (remove_unused_layers no) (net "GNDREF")))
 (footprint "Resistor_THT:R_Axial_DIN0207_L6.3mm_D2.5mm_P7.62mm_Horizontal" (layer "F.Cu") (at 138.115 65.69)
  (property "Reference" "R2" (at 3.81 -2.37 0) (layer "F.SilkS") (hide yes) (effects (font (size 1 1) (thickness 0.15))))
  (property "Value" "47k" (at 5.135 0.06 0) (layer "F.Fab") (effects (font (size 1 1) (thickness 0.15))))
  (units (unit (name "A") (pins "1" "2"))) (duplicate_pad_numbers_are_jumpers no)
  (fp_line (start 0.54 -1.37) (end 7.08 -1.37) (stroke (width 0.12) (type solid)) (layer "F.SilkS"))
  (fp_line (start 0.54 -1.04) (end 0.54 -1.37) (stroke (width 0.12) (type solid)) (layer "F.SilkS"))
  (fp_line (start 0.54 1.04) (end 0.54 1.37) (stroke (width 0.12) (type solid)) (layer "F.SilkS"))
  (fp_line (start 0.54 1.37) (end 7.08 1.37) (stroke (width 0.12) (type solid)) (layer "F.SilkS"))
  (fp_line (start 7.08 -1.37) (end 7.08 -1.04) (stroke (width 0.12) (type solid)) (layer "F.SilkS"))
  (fp_line (start 7.08 1.37) (end 7.08 1.04) (stroke (width 0.12) (type solid)) (layer "F.SilkS"))
  (pad "1" thru_hole circle (at 0 0) (size 1.6 1.6) (drill 0.8) (layers "*.Cu" "*.Mask") (remove_unused_layers no) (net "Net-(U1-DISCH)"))
  (pad "2" thru_hole circle (at 7.62 0) (size 1.6 1.6) (drill 0.8) (layers "*.Cu" "*.Mask") (remove_unused_layers no) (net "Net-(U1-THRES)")))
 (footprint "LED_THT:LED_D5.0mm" (layer "F.Cu") (at 148.96 69.5)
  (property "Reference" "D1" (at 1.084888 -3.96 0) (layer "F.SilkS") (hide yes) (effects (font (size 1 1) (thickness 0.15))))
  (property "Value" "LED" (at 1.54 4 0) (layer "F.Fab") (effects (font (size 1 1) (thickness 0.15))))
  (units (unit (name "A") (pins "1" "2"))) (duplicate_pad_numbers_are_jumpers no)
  (fp_line (start -1.29 -1.545) (end -1.29 1.545) (stroke (width 0.12) (type solid)) (layer "F.SilkS"))
  (fp_arc (start -1.29 -1.54483) (mid 2.071779 -2.880495) (end 4.26 0) (stroke (width 0.12) (type solid)) (layer "F.SilkS"))
  (fp_arc (start 4.26 0) (mid 2.071779 2.880495) (end -1.29 1.54483) (stroke (width 0.12) (type solid)) (layer "F.SilkS"))
  (fp_circle (center 1.27 0) (end 3.77 0) (stroke (width 0.12) (type solid)) (fill no) (layer "F.SilkS"))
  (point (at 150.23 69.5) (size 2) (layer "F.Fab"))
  (pad "1" thru_hole rect (at 0 0) (size 1.8 1.8) (drill 0.9) (layers "*.Cu" "*.Mask") (remove_unused_layers no) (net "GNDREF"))
  (pad "2" thru_hole circle (at 2.54 0) (size 1.8 1.8) (drill 0.9) (layers "*.Cu" "*.Mask") (remove_unused_layers no) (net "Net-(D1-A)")))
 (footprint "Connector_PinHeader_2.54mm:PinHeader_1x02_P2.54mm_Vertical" (layer "F.Cu") (at 155.235 64.46)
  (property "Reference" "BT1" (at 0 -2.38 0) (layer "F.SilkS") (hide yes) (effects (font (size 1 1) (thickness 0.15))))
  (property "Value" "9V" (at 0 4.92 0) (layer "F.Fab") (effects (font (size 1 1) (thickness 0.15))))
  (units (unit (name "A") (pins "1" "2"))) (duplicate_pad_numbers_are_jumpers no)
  (fp_line (start -1.38 -1.38) (end 0 -1.38) (stroke (width 0.12) (type solid)) (layer "F.SilkS"))
  (fp_line (start -1.38 0) (end -1.38 -1.38) (stroke (width 0.12) (type solid)) (layer "F.SilkS"))
  (fp_line (start -1.38 1.27) (end -1.38 3.92) (stroke (width 0.12) (type solid)) (layer "F.SilkS"))
  (fp_line (start -1.38 1.27) (end 1.38 1.27) (stroke (width 0.12) (type solid)) (layer "F.SilkS"))
  (fp_line (start -1.38 3.92) (end 1.38 3.92) (stroke (width 0.12) (type solid)) (layer "F.SilkS"))
  (fp_line (start 1.38 1.27) (end 1.38 3.92) (stroke (width 0.12) (type solid)) (layer "F.SilkS"))
  (pad "1" thru_hole rect (at 0 0) (size 1.7 1.7) (drill 1) (layers "*.Cu" "*.Mask") (remove_unused_layers no) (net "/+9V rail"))
  (pad "2" thru_hole circle (at 0 2.54) (size 1.7 1.7) (drill 1) (layers "*.Cu" "*.Mask") (remove_unused_layers no) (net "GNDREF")))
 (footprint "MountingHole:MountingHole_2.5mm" (layer "F.Cu") (at 123 60.25)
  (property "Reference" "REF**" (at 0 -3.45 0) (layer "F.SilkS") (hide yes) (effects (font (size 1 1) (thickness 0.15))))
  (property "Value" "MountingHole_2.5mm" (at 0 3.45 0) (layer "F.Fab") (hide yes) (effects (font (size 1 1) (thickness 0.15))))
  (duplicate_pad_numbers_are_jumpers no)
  (pad "" np_thru_hole circle (at 0 0) (size 0.5 0.5) (drill 2) (layers "*.Cu" "*.Mask")))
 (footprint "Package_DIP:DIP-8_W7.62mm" (layer "F.Cu") (at 127.425 61.66)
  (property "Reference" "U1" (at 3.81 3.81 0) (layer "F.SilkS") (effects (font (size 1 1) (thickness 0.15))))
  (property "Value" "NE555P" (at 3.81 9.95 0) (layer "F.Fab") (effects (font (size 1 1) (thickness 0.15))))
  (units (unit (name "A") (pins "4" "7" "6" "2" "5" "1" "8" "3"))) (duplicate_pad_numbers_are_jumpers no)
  (fp_line (start 1.16 -1.33) (end 1.16 8.95) (stroke (width 0.12) (type solid)) (layer "F.SilkS"))
  (fp_line (start 1.16 8.95) (end 6.46 8.95) (stroke (width 0.12) (type solid)) (layer "F.SilkS"))
  (fp_line (start 2.81 -1.33) (end 1.16 -1.33) (stroke (width 0.12) (type solid)) (layer "F.SilkS"))
  (fp_line (start 6.46 -1.33) (end 4.81 -1.33) (stroke (width 0.12) (type solid)) (layer "F.SilkS"))
  (fp_line (start 6.46 8.95) (end 6.46 -1.33) (stroke (width 0.12) (type solid)) (layer "F.SilkS"))
  (fp_arc (start 4.81 -1.33) (mid 3.81 -0.33) (end 2.81 -1.33) (stroke (width 0.12) (type solid)) (layer "F.SilkS"))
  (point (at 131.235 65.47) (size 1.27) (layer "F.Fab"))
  (pad "1" thru_hole roundrect (at 0 0) (size 1.6 1.6) (drill 0.8) (layers "*.Cu" "*.Mask") (remove_unused_layers no)
   (roundrect_rratio 0.15625) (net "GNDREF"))
  (pad "2" thru_hole circle (at 0 2.54) (size 1.6 1.6) (drill 0.8) (layers "*.Cu" "*.Mask") (remove_unused_layers no) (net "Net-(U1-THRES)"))
  (pad "3" thru_hole circle (at 0 5.08) (size 1.6 1.6) (drill 0.8) (layers "*.Cu" "*.Mask") (remove_unused_layers no) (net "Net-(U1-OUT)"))
  (pad "4" thru_hole circle (at 0 7.62) (size 1.6 1.6) (drill 0.8) (layers "*.Cu" "*.Mask") (remove_unused_layers no) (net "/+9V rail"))
  (pad "5" thru_hole circle (at 7.62 7.62) (size 1.6 1.6) (drill 0.8) (layers "*.Cu" "*.Mask") (remove_unused_layers no)
   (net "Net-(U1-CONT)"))
  (pad "6" thru_hole circle (at 7.62 5.08) (size 1.6 1.6) (drill 0.8) (layers "*.Cu" "*.Mask") (remove_unused_layers no)
   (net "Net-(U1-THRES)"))
  (pad "7" thru_hole circle (at 7.62 2.54) (size 1.6 1.6) (drill 0.8) (layers "*.Cu" "*.Mask") (remove_unused_layers no)
   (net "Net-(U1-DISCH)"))
  (pad "8" thru_hole circle (at 7.62 0) (size 1.6 1.6) (drill 0.8) (layers "*.Cu" "*.Mask") (remove_unused_layers no) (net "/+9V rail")))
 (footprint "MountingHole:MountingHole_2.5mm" (layer "F.Cu") (at 156.5 73)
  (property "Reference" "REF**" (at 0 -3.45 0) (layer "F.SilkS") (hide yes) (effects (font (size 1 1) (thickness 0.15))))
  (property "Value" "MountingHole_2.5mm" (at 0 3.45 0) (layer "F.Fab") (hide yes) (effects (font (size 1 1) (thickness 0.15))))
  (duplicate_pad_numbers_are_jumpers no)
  (pad "" np_thru_hole circle (at 0 0) (size 0.5 0.5) (drill 2) (layers "*.Cu" "*.Mask")))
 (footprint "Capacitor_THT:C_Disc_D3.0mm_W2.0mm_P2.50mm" (layer "F.Cu") (at 124 67 90)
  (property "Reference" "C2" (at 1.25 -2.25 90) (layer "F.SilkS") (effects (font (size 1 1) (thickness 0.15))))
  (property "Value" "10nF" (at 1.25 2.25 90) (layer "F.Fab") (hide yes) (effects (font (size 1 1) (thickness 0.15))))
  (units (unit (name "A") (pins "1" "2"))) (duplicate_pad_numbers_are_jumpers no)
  (fp_line (start 2.87 -1.12) (end 2.87 -0.972) (stroke (width 0.12) (type solid)) (layer "F.SilkS"))
  (fp_line (start -0.37 -1.12) (end 2.87 -1.12) (stroke (width 0.12) (type solid)) (layer "F.SilkS"))
  (fp_line (start -0.37 -0.972) (end -0.37 -1.12) (stroke (width 0.12) (type solid)) (layer "F.SilkS"))
  (fp_line (start 2.87 0.972) (end 2.87 1.12) (stroke (width 0.12) (type solid)) (layer "F.SilkS"))
  (fp_line (start 2.87 1.12) (end -0.37 1.12) (stroke (width 0.12) (type solid)) (layer "F.SilkS"))
  (fp_line (start -0.37 1.12) (end -0.37 0.972) (stroke (width 0.12) (type solid)) (layer "F.SilkS"))
  (pad "1" thru_hole circle (at 0 0 90) (size 1.6 1.6) (drill 0.8) (layers "*.Cu" "*.Mask") (remove_unused_layers no) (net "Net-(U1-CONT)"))
  (pad "2" thru_hole circle (at 2.5 0 90) (size 1.6 1.6) (drill 0.8) (layers "*.Cu" "*.Mask") (remove_unused_layers no) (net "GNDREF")))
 (gr_rect (start 120.25 56.75) (end 159.5 76) (stroke (width 0.05) (type default)) (fill no) (layer "Edge.Cuts"))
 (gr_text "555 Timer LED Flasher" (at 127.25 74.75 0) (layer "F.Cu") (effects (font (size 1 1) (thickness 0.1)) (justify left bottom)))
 (segment (start 138.115 59.385) (end 138.5 59) (width 0.2) (layer "F.Cu") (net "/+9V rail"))
 (segment (start 138.5 59) (end 151.25 59) (width 0.2) (layer "F.Cu") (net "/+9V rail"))
 (segment (start 155.235 62.985) (end 155.235 64.46) (width 0.2) (layer "F.Cu") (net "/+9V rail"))
 (segment (start 138.095 61.66) (end 138.115 61.64) (width 0.2) (layer "F.Cu") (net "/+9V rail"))
 (segment (start 138.115 61.64) (end 138.115 59.385) (width 0.2) (layer "F.Cu") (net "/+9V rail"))
 (segment (start 151.25 59) (end 155.235 62.985) (width 0.2) (layer "F.Cu") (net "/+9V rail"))
 (segment (start 135.045 61.66) (end 138.095 61.66) (width 0.2) (layer "F.Cu") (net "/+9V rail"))
 (segment (start 126.325 68.18) (end 126.325 60.875256) (width 0.2) (layer "B.Cu") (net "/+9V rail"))
 (segment (start 126.325 60.875256) (end 126.640256 60.56) (width 0.2) (layer "B.Cu") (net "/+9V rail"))
 (segment (start 133.945 60.56) (end 135.045 61.66) (width 0.2) (layer "B.Cu") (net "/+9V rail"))
 (segment (start 127.425 69.28) (end 126.325 68.18) (width 0.2) (layer "B.Cu") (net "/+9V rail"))
 (segment (start 126.640256 60.56) (end 133.945 60.56) (width 0.2) (layer "B.Cu") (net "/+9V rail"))
 (segment (start 155.235 67) (end 151.044888 62.809888) (width 0.2) (layer "F.Cu") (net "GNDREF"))
 (segment (start 149 74) (end 148.96 73.96) (width 0.2) (layer "F.Cu") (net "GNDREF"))
 (segment (start 148.96 73.96) (end 148.96 69.5) (width 0.2) (layer "F.Cu") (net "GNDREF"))
 (segment (start 155.235 67.765) (end 149 74) (width 0.2) (layer "F.Cu") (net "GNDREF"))
 (segment (start 124.585 64.5) (end 127.425 61.66) (width 0.2) (layer "F.Cu") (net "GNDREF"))
 (segment (start 151.044888 62.809888) (end 151.044888 62) (width 0.2) (layer "F.Cu") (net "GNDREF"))
 (segment (start 155.235 67) (end 155.235 67.765) (width 0.2) (layer "F.Cu") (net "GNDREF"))
 (segment (start 124 64.5) (end 124.585 64.5) (width 0.2) (layer "F.Cu") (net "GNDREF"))
 (segment (start 147.989365 69.5) (end 148.96 69.5) (width 0.2) (layer "B.Cu") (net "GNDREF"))
 (segment (start 127.425 61.66) (end 128.765 63) (width 0.2) (layer "B.Cu") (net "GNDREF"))
 (segment (start 141.489365 63) (end 147.989365 69.5) (width 0.2) (layer "B.Cu") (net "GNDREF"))
 (segment (start 128.765 63) (end 141.489365 63) (width 0.2) (layer "B.Cu") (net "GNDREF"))
 (segment (start 149.044888 62) (end 149.044888 62.380112) (width 0.2) (layer "F.Cu") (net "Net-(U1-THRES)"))
 (segment (start 143.925 67.5) (end 145.735 65.69) (width 0.2) (layer "F.Cu") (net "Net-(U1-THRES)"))
 (segment (start 149.044888 62.380112) (end 145.735 65.69) (width 0.2) (layer "F.Cu") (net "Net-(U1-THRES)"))
 (segment (start 132.505 64.2) (end 135.045 66.74) (width 0.2) (layer "F.Cu") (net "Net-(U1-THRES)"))
 (segment (start 135.045 66.74) (end 135.805 67.5) (width 0.2) (layer "F.Cu") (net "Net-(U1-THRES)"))
 (segment (start 135.805 67.5) (end 143.925 67.5) (width 0.2) (layer "F.Cu") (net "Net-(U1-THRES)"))
 (segment (start 127.425 64.2) (end 132.505 64.2) (width 0.2) (layer "F.Cu") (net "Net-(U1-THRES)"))
 (segment (start 124 67) (end 124 68.5) (width 0.2) (layer "F.Cu") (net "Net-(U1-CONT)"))
 (segment (start 134 72) (end 135.5 70.5) (width 0.2) (layer "F.Cu") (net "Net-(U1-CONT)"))
 (segment (start 124 68.5) (end 127.5 72) (width 0.2) (layer "F.Cu") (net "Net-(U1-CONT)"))
 (segment (start 127.5 72) (end 134 72) (width 0.2) (layer "F.Cu") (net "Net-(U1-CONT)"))
 (segment (start 135.5 70.5) (end 135.5 69.735) (width 0.2) (layer "F.Cu") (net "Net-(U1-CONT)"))
 (segment (start 135.5 69.735) (end 135.045 69.28) (width 0.2) (layer "F.Cu") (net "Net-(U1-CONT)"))
 (segment (start 145.735 69.74) (end 147.175 68.3) (width 0.2) (layer "F.Cu") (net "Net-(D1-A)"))
 (segment (start 150.3 68.3) (end 151.5 69.5) (width 0.2) (layer "F.Cu") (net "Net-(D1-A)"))
 (segment (start 147.175 68.3) (end 150.3 68.3) (width 0.2) (layer "F.Cu") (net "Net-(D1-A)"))
 (segment (start 128.865 68.18) (end 127.425 66.74) (width 0.2) (layer "F.Cu") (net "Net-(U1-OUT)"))
 (segment (start 136.555 68.18) (end 128.865 68.18) (width 0.2) (layer "F.Cu") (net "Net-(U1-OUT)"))
 (segment (start 138.115 69.74) (end 136.555 68.18) (width 0.2) (layer "F.Cu") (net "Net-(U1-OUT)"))
 (segment (start 138.115 65.69) (end 137.69 65.69) (width 0.2) (layer "F.Cu") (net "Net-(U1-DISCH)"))
 (segment (start 137.69 65.69) (end 136.2 64.2) (width 0.2) (layer "F.Cu") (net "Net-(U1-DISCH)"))
 (segment (start 145.735 61.64) (end 142.165 61.64) (width 0.2) (layer "F.Cu") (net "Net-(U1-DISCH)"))
 (segment (start 136.2 64.2) (end 135.045 64.2) (width 0.2) (layer "F.Cu") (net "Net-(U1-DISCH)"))
 (segment (start 142.165 61.64) (end 138.115 65.69) (width 0.2) (layer "F.Cu") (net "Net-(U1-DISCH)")))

